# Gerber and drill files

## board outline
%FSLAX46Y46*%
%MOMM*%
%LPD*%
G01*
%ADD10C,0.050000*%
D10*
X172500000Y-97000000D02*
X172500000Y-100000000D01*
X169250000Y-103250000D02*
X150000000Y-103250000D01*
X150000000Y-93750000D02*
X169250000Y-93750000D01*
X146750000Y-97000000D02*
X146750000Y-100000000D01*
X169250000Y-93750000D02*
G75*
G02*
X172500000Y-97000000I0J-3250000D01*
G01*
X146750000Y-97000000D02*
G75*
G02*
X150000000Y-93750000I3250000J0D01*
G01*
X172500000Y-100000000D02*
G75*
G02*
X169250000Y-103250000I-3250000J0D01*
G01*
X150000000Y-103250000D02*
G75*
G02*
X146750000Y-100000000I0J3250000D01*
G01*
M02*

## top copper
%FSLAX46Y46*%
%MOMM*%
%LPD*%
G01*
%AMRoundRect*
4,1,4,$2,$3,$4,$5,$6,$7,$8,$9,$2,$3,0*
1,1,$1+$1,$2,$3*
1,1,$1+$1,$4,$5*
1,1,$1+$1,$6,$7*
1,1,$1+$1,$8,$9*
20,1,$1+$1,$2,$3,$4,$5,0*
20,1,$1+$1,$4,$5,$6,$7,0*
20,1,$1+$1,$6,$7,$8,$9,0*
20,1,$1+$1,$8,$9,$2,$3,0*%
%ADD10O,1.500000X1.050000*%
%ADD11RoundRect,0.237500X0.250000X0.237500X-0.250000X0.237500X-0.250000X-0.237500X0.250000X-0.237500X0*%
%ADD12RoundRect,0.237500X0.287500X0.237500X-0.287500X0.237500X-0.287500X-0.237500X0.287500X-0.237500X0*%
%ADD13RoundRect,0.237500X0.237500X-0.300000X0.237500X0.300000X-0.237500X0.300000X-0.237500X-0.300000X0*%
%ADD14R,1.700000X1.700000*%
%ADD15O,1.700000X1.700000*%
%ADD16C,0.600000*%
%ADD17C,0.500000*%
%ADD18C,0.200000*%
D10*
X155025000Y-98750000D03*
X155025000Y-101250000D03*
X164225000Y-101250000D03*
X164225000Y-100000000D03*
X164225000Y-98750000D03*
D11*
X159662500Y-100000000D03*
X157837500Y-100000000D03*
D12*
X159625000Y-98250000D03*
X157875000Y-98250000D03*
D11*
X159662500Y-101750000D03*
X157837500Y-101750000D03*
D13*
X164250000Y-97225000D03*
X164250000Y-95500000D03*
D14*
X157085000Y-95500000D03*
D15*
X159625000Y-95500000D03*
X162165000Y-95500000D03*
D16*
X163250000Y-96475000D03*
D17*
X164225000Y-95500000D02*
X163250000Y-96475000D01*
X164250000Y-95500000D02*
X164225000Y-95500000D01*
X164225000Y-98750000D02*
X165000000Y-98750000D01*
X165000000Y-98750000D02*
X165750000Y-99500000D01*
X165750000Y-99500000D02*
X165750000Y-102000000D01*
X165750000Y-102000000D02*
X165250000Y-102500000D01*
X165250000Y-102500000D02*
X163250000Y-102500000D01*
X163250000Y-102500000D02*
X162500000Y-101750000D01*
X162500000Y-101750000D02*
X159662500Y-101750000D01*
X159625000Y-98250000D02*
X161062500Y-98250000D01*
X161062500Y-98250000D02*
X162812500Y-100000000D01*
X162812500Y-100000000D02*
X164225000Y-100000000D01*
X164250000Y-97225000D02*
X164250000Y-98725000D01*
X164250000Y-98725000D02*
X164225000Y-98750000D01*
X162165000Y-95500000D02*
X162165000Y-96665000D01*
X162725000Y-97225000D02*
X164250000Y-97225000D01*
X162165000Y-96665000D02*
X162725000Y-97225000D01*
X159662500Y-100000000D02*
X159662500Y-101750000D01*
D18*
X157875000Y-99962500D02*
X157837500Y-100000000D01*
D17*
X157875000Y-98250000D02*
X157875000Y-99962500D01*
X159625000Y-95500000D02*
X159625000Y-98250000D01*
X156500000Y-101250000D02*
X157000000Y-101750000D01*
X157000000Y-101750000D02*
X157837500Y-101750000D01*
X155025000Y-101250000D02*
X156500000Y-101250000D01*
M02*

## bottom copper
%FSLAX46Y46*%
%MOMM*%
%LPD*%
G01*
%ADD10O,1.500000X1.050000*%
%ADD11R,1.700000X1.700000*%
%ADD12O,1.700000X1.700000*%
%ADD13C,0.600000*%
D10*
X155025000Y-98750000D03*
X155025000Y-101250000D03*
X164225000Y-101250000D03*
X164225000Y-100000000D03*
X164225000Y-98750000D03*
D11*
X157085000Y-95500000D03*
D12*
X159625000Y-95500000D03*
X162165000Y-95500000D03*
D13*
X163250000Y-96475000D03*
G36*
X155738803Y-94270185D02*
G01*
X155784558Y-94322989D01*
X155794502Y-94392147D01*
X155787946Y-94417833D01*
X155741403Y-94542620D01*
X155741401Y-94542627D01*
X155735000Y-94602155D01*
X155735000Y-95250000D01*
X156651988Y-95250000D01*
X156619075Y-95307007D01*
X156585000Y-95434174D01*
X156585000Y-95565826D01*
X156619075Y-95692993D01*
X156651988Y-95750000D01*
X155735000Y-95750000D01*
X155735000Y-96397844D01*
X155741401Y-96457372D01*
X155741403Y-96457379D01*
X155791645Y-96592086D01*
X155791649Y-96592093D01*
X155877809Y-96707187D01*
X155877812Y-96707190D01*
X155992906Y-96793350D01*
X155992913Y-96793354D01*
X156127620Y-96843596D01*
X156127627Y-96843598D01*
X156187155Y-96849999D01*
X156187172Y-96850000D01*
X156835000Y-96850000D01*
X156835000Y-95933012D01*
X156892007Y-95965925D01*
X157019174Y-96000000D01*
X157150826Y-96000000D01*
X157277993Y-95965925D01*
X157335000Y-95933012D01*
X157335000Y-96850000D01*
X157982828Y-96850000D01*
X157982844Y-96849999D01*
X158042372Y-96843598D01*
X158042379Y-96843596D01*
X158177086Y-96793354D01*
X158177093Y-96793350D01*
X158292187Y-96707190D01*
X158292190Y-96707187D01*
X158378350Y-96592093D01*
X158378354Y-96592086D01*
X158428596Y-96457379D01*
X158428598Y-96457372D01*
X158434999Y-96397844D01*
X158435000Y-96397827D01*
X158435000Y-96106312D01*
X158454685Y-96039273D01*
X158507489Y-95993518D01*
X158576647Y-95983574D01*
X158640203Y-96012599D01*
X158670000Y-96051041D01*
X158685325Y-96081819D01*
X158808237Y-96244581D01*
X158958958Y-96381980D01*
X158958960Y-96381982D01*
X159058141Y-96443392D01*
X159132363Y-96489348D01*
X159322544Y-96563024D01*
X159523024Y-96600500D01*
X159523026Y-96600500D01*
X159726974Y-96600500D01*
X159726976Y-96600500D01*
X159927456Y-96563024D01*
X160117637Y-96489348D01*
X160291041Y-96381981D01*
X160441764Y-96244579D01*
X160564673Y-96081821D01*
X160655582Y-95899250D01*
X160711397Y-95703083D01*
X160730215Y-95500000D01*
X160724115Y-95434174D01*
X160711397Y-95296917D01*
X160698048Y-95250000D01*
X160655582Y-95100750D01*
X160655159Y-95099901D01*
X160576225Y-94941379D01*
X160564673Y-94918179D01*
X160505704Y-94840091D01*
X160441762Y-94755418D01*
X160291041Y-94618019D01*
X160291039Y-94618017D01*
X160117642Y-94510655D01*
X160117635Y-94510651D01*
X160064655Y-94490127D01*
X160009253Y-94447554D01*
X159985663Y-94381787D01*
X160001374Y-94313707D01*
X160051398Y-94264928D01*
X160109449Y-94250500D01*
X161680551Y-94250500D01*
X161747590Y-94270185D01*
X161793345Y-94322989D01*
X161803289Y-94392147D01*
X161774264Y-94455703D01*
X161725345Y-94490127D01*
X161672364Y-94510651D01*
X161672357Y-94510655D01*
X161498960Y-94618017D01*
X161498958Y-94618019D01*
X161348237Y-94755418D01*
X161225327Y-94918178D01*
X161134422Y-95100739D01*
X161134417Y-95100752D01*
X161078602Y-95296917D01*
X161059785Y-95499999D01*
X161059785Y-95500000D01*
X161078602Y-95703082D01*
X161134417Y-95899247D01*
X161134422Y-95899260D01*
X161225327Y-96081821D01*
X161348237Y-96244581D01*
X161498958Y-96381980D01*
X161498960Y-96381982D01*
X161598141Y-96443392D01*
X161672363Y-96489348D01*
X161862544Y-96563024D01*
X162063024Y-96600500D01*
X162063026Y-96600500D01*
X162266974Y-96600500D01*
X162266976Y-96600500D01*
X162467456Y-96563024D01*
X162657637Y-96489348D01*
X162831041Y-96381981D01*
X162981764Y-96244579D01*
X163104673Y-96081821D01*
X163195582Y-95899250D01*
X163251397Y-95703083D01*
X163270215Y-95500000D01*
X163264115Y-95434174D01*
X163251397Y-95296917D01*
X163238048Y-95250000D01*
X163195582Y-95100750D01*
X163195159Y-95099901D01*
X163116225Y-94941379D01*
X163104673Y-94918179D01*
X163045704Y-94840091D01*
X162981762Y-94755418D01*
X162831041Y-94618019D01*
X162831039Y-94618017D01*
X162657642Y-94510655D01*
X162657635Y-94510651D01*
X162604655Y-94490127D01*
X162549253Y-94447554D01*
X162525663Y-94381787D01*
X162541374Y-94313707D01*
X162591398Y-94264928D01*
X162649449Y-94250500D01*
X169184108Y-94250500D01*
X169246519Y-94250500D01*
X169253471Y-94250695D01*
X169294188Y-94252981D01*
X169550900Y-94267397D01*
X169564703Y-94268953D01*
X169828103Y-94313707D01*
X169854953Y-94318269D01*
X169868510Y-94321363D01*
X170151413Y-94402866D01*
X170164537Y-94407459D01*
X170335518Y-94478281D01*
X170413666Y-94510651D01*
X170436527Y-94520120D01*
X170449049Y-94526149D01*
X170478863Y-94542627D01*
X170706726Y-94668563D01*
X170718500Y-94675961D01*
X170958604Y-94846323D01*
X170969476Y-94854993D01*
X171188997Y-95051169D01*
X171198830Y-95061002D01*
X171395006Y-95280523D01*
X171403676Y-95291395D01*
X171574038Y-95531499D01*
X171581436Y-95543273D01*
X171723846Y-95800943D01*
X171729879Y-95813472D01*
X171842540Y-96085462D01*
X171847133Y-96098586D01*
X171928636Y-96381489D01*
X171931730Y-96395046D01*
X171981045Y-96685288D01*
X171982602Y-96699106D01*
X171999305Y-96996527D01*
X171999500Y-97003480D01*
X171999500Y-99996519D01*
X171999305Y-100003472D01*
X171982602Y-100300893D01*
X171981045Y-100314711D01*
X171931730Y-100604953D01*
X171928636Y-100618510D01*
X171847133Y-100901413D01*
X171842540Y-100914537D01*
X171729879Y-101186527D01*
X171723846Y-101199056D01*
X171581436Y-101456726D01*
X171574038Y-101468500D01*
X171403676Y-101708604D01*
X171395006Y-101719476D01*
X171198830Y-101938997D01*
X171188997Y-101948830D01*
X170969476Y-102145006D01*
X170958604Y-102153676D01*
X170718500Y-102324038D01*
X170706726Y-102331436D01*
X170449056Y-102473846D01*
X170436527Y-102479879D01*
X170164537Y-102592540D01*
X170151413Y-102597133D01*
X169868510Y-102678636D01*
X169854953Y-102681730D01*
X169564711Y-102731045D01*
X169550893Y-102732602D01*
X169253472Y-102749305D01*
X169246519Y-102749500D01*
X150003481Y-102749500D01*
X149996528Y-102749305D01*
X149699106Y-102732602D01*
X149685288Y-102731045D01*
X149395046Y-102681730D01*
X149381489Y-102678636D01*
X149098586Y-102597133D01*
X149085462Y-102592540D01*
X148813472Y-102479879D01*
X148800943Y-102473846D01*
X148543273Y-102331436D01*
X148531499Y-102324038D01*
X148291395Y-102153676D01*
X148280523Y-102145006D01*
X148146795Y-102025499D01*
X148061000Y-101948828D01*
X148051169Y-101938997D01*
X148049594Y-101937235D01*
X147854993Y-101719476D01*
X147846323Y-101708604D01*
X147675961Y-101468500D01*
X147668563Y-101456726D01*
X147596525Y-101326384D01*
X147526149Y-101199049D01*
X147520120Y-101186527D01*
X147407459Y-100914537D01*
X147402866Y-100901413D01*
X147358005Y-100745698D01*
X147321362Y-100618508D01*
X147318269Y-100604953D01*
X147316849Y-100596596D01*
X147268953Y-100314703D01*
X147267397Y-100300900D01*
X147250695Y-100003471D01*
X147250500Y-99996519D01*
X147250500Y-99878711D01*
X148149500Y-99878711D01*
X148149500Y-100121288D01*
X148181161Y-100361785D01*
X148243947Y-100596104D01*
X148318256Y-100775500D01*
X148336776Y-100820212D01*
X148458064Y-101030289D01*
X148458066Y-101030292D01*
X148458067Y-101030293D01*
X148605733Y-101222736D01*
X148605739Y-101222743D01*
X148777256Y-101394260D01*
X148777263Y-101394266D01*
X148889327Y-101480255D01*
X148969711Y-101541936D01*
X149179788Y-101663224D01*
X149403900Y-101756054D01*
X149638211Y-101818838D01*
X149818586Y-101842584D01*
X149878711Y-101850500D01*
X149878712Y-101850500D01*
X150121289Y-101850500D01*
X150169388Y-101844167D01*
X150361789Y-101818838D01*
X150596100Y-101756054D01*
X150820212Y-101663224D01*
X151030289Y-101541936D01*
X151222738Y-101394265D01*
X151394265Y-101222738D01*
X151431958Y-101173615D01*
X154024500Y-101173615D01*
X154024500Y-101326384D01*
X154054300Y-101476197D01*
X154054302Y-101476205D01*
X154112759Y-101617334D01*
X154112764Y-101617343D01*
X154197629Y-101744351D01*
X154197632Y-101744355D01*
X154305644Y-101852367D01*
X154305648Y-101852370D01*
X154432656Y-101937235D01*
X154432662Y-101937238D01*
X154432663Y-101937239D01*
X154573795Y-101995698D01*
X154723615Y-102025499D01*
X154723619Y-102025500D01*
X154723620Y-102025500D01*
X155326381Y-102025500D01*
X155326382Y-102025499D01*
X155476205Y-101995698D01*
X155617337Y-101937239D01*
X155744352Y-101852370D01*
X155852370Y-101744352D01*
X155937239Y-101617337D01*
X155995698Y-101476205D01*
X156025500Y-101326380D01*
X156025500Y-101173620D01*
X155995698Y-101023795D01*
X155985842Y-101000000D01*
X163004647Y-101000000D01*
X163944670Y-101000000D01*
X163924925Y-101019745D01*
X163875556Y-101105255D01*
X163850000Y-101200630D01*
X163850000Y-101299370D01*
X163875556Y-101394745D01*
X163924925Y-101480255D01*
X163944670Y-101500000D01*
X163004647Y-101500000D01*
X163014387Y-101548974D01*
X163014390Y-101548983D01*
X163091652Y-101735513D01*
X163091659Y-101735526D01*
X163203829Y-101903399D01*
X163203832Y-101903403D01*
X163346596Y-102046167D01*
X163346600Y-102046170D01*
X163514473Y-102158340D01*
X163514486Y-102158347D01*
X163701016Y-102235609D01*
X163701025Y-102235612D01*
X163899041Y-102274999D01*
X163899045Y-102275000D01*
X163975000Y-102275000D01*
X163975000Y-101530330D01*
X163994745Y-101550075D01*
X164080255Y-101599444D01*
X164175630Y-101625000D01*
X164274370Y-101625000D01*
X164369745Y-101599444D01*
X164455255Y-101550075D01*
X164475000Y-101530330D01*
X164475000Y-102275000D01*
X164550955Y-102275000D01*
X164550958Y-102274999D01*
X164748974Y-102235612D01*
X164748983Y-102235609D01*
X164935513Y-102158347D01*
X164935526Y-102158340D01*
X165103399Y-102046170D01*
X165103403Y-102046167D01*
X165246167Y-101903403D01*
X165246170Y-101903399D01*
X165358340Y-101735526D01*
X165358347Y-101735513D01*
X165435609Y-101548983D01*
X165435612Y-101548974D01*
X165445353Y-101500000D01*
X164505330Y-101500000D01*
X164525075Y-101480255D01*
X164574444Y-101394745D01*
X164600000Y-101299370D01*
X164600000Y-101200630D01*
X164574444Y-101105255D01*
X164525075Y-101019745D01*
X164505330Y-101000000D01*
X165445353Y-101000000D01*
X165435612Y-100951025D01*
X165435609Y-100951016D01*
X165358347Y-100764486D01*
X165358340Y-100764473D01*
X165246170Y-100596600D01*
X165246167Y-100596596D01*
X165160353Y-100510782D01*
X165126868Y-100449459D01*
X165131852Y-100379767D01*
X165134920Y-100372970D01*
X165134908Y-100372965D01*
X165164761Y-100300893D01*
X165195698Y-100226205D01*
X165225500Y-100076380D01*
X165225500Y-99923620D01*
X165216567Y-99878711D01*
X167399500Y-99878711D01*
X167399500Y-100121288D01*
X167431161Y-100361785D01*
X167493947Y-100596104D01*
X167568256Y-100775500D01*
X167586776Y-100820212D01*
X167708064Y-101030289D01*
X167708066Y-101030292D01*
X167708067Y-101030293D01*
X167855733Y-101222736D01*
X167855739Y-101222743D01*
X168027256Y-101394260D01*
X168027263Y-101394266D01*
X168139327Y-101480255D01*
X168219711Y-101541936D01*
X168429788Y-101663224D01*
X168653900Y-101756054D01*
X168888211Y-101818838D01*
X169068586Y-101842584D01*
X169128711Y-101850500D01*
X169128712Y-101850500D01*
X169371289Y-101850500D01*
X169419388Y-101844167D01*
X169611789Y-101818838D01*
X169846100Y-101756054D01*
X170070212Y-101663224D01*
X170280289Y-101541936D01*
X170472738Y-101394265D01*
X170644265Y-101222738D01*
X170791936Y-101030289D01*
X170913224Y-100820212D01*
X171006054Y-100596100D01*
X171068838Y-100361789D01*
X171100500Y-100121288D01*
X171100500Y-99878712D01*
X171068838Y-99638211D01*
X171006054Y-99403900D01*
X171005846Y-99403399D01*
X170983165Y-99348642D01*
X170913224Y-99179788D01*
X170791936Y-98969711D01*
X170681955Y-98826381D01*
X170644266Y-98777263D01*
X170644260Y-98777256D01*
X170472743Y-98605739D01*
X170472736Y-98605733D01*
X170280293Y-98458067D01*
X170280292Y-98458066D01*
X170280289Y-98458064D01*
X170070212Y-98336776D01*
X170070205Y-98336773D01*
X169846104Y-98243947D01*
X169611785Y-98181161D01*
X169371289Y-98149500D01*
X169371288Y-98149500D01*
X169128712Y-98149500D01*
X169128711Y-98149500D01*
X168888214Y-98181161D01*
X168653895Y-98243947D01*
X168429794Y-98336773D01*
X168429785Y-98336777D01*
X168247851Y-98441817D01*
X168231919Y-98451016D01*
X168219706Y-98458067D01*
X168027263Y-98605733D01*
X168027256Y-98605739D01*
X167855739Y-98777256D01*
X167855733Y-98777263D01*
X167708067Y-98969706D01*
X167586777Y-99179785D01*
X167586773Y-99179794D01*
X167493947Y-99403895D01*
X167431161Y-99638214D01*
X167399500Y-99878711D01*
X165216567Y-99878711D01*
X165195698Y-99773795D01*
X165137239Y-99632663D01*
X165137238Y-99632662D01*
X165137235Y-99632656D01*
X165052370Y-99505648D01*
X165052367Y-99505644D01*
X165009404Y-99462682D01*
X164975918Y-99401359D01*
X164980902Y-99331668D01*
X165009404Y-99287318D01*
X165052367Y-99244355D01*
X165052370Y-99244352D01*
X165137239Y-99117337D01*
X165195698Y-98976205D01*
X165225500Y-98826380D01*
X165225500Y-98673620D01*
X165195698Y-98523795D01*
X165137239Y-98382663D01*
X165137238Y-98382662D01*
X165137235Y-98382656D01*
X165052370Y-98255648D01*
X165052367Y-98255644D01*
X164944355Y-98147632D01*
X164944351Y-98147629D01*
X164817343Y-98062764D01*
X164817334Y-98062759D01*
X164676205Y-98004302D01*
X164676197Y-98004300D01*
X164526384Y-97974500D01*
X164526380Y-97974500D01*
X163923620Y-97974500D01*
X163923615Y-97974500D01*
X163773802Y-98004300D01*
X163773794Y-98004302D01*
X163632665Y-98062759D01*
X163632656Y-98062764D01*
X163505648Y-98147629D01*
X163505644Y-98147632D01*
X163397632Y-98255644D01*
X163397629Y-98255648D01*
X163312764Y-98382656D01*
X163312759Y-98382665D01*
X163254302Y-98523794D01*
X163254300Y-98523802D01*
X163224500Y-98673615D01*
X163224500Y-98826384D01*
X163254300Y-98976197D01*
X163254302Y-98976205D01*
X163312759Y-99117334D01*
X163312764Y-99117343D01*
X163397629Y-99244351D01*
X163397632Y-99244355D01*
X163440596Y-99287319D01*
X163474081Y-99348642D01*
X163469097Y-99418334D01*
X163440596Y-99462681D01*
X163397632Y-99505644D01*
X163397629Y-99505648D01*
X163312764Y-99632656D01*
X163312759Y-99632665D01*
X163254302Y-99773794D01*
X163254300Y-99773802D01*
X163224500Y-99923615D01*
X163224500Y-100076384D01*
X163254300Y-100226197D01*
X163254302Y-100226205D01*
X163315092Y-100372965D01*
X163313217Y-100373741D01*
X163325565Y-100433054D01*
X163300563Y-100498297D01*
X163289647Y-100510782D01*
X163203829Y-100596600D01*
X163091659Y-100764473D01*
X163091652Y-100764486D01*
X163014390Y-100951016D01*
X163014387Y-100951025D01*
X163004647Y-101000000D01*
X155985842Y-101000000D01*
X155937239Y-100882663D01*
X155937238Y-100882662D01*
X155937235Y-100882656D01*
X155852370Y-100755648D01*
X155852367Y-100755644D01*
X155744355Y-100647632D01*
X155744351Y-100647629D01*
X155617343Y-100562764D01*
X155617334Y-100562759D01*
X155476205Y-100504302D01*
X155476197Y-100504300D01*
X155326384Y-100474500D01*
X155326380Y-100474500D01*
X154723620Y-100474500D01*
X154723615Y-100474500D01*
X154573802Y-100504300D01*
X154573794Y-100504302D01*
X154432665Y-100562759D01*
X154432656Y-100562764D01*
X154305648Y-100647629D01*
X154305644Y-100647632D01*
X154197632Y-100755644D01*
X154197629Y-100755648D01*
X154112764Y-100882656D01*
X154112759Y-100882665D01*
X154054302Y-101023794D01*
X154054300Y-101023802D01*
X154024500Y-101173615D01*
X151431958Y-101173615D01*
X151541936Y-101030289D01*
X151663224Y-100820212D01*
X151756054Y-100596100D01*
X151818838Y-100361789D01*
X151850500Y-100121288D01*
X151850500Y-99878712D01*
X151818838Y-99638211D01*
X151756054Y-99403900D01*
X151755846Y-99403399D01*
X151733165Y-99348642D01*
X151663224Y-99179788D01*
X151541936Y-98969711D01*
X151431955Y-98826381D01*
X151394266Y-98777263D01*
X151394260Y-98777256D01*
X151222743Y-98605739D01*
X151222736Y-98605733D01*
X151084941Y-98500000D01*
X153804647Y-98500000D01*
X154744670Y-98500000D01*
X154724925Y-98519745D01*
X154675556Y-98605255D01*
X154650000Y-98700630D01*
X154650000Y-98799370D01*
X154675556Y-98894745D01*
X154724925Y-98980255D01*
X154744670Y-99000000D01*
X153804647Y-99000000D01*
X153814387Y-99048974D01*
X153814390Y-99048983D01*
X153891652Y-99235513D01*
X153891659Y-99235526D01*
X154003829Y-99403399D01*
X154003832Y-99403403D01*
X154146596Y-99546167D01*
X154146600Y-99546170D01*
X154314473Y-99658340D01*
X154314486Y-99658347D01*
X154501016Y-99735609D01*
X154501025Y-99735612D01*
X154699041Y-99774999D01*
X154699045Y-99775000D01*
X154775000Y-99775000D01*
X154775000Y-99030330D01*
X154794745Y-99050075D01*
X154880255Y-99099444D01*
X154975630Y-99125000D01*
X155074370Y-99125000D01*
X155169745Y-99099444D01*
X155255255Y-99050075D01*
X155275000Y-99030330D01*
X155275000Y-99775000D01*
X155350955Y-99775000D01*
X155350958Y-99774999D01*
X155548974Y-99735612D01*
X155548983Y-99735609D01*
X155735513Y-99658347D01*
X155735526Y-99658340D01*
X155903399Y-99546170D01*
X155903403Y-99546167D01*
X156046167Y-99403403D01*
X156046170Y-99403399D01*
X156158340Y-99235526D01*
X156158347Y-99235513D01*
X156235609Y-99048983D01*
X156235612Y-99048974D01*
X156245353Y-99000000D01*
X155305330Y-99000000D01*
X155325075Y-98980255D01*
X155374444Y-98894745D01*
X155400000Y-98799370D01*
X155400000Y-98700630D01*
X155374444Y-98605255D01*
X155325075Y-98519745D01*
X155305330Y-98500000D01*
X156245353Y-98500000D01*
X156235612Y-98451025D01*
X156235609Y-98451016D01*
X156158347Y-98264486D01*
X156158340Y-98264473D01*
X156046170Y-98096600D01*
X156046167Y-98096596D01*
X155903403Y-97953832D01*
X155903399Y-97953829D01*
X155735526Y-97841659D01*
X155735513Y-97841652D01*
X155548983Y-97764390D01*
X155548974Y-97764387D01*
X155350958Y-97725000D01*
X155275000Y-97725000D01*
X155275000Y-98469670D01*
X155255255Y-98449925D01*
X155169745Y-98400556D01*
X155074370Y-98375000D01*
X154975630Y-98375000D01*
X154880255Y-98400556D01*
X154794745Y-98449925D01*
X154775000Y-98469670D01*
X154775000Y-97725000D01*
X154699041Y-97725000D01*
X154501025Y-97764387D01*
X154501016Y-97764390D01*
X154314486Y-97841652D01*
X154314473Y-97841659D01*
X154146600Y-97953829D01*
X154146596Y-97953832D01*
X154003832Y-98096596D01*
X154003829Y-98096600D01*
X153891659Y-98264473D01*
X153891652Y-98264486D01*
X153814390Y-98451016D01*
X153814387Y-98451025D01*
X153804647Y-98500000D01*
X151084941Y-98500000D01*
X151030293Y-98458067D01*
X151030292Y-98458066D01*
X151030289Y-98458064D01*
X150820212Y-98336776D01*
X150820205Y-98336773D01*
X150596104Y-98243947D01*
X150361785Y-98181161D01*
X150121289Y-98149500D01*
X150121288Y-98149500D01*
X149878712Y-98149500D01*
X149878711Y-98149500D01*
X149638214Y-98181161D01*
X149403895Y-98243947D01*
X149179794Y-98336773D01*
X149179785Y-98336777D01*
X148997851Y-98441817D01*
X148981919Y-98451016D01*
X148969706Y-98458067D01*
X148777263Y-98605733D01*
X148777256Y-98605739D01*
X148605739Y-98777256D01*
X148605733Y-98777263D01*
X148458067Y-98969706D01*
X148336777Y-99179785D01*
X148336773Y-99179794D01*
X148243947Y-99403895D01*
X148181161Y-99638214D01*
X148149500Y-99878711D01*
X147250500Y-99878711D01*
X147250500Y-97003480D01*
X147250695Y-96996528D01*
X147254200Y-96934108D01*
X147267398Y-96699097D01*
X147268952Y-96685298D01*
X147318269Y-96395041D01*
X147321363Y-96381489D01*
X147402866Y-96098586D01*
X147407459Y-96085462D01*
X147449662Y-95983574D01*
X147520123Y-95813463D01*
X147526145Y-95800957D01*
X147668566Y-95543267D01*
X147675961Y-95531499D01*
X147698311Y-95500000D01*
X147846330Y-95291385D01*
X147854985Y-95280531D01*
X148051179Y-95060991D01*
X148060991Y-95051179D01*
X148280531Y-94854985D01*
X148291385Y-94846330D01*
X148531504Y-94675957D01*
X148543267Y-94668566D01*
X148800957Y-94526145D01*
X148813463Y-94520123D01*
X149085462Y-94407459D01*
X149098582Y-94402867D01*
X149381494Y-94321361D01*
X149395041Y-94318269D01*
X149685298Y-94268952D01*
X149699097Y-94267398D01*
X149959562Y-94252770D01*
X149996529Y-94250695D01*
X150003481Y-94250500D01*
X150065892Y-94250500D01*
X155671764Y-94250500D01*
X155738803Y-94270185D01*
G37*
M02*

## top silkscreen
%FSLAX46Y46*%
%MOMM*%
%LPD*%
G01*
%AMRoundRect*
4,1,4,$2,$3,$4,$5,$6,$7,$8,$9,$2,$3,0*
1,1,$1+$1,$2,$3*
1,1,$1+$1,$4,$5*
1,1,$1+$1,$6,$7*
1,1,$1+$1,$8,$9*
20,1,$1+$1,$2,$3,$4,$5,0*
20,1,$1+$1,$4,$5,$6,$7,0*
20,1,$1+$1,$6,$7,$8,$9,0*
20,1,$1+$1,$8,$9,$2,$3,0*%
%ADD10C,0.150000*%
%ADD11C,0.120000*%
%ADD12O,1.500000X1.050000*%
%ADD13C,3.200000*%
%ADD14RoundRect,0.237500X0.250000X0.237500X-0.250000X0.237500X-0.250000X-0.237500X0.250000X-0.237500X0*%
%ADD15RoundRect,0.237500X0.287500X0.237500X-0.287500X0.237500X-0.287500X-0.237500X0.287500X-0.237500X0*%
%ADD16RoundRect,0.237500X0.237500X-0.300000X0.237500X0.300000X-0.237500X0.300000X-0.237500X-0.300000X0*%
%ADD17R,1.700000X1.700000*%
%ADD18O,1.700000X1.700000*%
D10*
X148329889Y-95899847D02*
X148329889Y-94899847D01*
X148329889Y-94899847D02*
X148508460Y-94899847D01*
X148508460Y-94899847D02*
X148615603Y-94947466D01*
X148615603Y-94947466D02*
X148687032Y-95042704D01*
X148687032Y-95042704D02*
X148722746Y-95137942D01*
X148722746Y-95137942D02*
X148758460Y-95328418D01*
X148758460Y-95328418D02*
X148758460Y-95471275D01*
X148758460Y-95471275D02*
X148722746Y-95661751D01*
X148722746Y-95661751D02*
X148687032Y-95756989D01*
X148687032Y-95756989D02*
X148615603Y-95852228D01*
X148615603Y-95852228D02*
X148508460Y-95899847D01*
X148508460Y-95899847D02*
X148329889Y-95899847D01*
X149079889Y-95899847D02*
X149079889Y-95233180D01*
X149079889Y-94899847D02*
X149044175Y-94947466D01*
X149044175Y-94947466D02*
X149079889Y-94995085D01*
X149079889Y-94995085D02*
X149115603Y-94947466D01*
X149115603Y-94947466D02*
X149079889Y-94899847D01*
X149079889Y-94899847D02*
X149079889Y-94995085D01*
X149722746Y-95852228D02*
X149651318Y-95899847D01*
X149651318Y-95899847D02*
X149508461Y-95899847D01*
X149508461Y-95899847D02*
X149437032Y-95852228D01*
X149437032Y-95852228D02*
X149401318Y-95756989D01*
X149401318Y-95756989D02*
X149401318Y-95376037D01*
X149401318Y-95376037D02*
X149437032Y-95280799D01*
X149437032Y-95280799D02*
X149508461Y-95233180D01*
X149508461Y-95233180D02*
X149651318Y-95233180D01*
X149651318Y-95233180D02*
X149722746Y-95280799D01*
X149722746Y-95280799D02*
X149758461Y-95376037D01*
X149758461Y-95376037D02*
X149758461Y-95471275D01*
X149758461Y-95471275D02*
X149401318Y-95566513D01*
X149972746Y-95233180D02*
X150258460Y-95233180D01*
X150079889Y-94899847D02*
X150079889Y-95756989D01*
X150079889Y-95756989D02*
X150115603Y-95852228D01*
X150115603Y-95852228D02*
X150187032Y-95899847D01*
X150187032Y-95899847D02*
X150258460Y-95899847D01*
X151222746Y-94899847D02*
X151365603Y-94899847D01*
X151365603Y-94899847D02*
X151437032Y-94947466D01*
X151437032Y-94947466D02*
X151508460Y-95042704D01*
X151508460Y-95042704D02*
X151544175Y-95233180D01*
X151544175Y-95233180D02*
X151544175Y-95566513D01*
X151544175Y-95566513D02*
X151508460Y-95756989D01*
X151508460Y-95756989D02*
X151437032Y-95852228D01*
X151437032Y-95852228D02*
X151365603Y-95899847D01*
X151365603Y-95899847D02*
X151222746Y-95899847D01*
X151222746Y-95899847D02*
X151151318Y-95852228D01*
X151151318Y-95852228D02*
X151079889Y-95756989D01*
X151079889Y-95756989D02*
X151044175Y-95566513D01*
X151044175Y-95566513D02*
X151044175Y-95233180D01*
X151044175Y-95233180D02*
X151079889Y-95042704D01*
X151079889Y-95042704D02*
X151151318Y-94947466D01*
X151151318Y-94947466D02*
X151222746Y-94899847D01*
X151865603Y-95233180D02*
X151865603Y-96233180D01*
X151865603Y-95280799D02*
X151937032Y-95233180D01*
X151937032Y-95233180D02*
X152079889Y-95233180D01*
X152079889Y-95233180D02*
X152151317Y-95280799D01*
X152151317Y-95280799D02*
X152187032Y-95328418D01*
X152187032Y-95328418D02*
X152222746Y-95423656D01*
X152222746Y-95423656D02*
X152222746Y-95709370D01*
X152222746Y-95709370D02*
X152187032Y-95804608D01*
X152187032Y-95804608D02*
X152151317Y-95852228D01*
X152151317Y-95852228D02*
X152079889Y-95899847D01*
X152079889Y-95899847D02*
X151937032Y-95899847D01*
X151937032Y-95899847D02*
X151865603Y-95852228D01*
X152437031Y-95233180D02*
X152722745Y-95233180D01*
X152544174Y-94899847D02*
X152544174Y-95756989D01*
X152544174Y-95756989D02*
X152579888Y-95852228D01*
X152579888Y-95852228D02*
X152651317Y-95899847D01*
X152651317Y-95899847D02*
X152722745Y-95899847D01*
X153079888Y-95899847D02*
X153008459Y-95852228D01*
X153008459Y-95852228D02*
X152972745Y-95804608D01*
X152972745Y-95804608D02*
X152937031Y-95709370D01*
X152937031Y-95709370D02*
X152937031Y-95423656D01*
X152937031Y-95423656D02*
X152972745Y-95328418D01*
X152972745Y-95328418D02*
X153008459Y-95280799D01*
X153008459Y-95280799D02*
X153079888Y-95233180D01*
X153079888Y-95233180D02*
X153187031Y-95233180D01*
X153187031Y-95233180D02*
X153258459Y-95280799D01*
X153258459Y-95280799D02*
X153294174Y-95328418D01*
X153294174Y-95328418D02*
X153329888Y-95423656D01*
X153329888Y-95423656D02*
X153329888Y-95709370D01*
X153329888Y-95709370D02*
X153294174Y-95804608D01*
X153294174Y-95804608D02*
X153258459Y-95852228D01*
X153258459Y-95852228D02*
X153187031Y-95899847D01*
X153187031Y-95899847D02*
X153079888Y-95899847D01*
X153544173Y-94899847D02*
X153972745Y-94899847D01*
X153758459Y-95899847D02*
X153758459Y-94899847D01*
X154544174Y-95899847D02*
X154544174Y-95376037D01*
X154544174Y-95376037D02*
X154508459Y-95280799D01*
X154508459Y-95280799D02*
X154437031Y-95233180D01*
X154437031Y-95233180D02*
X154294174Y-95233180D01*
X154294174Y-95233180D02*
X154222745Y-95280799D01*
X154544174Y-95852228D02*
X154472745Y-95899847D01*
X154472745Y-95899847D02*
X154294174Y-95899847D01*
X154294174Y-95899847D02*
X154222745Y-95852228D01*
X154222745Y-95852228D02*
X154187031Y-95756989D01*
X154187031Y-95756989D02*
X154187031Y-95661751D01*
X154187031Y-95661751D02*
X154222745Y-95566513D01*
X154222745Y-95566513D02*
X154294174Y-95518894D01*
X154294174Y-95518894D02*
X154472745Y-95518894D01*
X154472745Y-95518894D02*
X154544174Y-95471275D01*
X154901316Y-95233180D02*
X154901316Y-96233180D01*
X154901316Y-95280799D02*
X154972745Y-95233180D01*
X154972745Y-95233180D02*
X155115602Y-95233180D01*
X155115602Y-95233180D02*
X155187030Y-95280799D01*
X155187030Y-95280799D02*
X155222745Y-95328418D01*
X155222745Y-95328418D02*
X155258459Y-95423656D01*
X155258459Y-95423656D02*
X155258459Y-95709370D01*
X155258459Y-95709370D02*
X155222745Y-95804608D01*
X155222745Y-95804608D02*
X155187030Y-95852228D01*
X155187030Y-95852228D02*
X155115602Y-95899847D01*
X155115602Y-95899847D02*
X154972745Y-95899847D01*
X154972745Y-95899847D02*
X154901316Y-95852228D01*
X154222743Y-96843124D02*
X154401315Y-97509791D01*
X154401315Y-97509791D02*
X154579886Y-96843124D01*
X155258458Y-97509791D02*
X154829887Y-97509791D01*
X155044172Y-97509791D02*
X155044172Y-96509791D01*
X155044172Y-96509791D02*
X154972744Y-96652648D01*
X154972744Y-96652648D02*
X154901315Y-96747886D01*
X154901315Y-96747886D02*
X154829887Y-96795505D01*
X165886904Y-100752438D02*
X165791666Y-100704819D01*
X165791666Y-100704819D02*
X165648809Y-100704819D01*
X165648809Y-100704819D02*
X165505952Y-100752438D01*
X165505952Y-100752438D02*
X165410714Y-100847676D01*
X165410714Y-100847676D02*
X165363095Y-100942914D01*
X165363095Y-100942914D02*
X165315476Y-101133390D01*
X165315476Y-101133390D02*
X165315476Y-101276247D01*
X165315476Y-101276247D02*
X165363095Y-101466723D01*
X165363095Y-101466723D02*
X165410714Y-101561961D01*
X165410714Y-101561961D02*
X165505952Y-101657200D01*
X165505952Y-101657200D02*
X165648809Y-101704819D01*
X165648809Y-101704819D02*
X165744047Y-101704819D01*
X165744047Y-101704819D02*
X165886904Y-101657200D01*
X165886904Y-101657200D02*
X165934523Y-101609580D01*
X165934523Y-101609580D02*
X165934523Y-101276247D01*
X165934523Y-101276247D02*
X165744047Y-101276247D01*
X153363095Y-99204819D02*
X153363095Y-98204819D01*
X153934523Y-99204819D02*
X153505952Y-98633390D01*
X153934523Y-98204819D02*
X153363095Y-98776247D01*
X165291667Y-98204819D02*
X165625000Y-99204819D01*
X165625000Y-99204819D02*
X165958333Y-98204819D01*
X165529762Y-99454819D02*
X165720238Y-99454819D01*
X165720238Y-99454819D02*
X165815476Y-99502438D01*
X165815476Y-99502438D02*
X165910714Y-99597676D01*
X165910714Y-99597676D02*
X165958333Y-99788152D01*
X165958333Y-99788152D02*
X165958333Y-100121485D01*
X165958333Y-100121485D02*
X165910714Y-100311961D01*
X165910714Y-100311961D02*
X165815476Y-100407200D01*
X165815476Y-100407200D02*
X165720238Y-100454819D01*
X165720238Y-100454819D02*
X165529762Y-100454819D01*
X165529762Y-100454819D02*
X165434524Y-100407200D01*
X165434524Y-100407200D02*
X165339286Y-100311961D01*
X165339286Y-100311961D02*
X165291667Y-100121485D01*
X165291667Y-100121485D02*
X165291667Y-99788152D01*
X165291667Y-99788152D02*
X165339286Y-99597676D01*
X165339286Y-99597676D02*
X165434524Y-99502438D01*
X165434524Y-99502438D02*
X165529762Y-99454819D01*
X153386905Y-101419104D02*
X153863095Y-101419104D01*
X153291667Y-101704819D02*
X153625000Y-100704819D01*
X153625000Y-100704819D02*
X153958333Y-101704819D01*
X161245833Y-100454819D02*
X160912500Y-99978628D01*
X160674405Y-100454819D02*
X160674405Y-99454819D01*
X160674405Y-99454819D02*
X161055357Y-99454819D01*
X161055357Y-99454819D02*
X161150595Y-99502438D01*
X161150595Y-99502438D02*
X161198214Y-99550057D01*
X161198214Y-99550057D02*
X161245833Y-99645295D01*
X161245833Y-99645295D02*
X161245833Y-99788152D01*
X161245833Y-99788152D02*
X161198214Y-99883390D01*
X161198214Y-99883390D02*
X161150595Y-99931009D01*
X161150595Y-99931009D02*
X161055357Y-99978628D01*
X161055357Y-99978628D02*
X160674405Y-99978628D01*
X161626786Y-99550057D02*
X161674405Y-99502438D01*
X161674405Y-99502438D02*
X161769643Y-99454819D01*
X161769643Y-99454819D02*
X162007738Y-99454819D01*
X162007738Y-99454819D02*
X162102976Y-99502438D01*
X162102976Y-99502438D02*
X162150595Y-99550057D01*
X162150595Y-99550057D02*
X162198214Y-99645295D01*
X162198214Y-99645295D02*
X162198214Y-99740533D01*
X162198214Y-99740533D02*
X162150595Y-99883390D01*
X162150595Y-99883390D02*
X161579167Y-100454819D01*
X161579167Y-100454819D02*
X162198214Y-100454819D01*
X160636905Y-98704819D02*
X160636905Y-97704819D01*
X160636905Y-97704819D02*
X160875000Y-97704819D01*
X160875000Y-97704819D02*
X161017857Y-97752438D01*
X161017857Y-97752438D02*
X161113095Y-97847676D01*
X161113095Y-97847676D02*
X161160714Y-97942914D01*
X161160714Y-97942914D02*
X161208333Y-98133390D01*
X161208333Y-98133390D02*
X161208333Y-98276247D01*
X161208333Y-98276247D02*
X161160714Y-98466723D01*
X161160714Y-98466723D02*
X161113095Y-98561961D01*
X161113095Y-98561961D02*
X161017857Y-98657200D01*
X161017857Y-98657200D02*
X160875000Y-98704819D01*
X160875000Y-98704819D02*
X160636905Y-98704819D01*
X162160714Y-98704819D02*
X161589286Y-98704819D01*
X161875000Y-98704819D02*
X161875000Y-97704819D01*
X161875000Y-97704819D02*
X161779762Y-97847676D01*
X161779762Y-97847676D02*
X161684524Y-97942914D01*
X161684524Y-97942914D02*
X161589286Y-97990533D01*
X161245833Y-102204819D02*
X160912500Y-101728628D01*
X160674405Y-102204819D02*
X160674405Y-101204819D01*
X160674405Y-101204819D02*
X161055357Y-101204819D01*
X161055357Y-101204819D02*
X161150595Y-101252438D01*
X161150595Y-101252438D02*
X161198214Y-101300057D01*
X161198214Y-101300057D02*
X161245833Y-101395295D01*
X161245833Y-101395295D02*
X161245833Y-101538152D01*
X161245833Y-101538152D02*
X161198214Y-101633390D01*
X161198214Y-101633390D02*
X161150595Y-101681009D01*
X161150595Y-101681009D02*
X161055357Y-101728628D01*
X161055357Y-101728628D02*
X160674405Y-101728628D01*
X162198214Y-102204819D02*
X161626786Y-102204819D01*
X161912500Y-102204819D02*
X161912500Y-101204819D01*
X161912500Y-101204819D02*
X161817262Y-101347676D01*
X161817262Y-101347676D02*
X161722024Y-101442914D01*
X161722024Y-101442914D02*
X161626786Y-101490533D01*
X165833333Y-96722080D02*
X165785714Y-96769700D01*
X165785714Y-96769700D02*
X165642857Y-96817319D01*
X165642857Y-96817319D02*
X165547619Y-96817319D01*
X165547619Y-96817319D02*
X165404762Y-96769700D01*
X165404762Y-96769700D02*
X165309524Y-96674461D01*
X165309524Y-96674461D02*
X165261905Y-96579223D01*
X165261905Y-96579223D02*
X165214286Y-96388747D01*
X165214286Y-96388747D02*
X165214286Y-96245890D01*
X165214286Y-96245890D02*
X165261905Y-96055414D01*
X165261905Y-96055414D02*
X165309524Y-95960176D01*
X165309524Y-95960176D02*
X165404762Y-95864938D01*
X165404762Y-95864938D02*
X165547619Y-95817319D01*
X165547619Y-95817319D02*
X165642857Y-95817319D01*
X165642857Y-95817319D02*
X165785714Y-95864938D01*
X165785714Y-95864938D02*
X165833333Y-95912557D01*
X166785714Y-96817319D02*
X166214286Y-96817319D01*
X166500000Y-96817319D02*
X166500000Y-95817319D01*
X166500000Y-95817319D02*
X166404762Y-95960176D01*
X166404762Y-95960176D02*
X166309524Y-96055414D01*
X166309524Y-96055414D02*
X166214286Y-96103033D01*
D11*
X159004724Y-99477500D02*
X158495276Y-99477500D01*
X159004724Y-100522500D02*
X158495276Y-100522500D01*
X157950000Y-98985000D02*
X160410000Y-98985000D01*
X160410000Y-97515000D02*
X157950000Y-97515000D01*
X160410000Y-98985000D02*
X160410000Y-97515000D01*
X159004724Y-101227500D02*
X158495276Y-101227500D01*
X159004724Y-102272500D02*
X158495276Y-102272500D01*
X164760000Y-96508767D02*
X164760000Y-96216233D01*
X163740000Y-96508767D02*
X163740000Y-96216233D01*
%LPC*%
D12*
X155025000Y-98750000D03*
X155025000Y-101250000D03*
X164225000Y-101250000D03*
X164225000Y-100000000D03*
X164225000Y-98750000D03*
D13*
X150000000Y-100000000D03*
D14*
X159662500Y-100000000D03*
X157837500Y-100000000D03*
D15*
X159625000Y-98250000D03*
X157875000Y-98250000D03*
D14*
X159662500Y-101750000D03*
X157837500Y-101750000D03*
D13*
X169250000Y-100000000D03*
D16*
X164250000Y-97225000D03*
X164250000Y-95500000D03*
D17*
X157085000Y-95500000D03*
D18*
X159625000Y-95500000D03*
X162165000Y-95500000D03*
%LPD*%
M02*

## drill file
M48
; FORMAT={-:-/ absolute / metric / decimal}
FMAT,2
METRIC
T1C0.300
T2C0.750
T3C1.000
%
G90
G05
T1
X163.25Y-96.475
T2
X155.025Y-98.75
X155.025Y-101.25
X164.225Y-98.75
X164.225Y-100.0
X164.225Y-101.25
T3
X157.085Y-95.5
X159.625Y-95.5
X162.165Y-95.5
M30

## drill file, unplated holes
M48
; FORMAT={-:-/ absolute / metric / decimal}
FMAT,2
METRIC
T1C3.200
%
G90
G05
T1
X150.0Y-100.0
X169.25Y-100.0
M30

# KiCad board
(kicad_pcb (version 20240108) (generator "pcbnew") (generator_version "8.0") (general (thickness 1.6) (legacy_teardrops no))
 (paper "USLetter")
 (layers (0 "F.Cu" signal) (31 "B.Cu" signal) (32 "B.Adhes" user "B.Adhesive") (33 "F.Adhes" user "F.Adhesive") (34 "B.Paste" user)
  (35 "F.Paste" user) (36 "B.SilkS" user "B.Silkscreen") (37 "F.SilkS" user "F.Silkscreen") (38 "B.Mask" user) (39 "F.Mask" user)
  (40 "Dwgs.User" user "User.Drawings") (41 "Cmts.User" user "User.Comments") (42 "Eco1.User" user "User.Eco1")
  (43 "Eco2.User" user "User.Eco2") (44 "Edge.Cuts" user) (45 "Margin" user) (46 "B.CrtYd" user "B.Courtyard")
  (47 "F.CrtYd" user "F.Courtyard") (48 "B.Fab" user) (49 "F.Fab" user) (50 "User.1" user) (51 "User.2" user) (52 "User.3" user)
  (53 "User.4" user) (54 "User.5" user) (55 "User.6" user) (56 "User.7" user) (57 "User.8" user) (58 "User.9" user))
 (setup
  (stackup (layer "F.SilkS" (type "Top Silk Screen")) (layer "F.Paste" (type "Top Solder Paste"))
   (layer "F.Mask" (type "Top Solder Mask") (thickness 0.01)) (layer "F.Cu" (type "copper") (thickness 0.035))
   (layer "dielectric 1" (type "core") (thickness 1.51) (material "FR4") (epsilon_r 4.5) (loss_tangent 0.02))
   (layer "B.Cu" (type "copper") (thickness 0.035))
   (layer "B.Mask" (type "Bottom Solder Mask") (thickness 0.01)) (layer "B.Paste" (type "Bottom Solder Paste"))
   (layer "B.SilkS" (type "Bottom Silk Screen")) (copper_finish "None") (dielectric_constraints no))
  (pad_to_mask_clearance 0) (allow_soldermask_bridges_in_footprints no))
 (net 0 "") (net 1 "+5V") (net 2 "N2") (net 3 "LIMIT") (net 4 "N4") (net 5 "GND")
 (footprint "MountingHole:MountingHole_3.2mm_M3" (layer "F.Cu") (at 150 100)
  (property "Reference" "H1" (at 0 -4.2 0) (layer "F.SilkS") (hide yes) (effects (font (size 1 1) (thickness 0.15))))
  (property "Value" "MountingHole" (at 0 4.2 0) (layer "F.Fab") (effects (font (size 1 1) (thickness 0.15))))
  (pad "" np_thru_hole circle (at 0 0) (size 3.2 3.2) (drill 3.2) (layers "F&B.Cu" "*.Mask")))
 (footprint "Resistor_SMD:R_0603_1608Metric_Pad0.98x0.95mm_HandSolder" (layer "F.Cu") (at 158.75 100 180)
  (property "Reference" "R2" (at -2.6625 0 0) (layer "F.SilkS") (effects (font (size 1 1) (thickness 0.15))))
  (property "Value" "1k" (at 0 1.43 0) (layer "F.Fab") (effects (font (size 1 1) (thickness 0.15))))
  (fp_line (start -0.254724 0.5225) (end 0.254724 0.5225) (stroke (width 0.12) (type solid)) (layer "F.SilkS"))
  (fp_line (start -0.254724 -0.5225) (end 0.254724 -0.5225) (stroke (width 0.12) (type solid)) (layer "F.SilkS"))
  (pad "1" smd roundrect (at -0.9125 0 180) (size 0.975 0.95) (layers "F.Cu" "F.Paste" "F.Mask") (roundrect_rratio 0.25) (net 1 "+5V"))
  (pad "2" smd roundrect (at 0.9125 0 180) (size 0.975 0.95) (layers "F.Cu" "F.Paste" "F.Mask") (roundrect_rratio 0.25) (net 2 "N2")))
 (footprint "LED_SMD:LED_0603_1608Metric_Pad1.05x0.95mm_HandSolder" (layer "F.Cu") (at 158.75 98.25 180)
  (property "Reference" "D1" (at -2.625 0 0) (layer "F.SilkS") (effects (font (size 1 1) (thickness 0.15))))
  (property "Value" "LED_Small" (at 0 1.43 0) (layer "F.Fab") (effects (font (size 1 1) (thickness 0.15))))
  (fp_line (start 0.8 -0.735) (end -1.66 -0.735) (stroke (width 0.12) (type solid)) (layer "F.SilkS"))
  (fp_line (start -1.66 0.735) (end 0.8 0.735) (stroke (width 0.12) (type solid)) (layer "F.SilkS"))
  (fp_line (start -1.66 -0.735) (end -1.66 0.735) (stroke (width 0.12) (type solid)) (layer "F.SilkS"))
  (pad "1" smd roundrect (at -0.875 0 180) (size 1.05 0.95) (layers "F.Cu" "F.Paste" "F.Mask") (roundrect_rratio 0.25) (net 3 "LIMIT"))
  (pad "2" smd roundrect (at 0.875 0 180) (size 1.05 0.95) (layers "F.Cu" "F.Paste" "F.Mask") (roundrect_rratio 0.25) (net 2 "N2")))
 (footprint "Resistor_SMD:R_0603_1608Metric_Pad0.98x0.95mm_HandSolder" (layer "F.Cu") (at 158.75 101.75 180)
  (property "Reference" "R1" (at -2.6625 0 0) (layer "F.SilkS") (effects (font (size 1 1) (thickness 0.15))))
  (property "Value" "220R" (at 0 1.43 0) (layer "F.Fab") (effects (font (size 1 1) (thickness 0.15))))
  (fp_line (start -0.254724 0.5225) (end 0.254724 0.5225) (stroke (width 0.12) (type solid)) (layer "F.SilkS"))
  (fp_line (start -0.254724 -0.5225) (end 0.254724 -0.5225) (stroke (width 0.12) (type solid)) (layer "F.SilkS"))
  (pad "1" smd roundrect (at -0.9125 0 180) (size 0.975 0.95) (layers "F.Cu" "F.Paste" "F.Mask") (roundrect_rratio 0.25) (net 1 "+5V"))
  (pad "2" smd roundrect (at 0.9125 0 180) (size 0.975 0.95) (layers "F.Cu" "F.Paste" "F.Mask") (roundrect_rratio 0.25) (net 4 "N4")))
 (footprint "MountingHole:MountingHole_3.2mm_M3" (layer "F.Cu") (at 169.25 100)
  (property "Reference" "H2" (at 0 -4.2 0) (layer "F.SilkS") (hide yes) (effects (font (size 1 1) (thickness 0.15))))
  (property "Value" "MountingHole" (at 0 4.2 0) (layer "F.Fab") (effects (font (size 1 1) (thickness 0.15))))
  (pad "" np_thru_hole circle (at 0 0) (size 3.2 3.2) (drill 3.2) (layers "F&B.Cu" "*.Mask")))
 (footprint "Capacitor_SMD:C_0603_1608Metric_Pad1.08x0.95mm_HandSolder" (layer "F.Cu") (at 164.25 96.3625 90)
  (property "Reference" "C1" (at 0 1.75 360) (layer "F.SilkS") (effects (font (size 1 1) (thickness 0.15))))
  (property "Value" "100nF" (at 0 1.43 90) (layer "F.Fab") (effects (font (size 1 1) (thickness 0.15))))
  (fp_line (start -0.146267 -0.51) (end 0.146267 -0.51) (stroke (width 0.12) (type solid)) (layer "F.SilkS"))
  (fp_line (start -0.146267 0.51) (end 0.146267 0.51) (stroke (width 0.12) (type solid)) (layer "F.SilkS"))
  (pad "1" smd roundrect (at -0.8625 0 90) (size 1.075 0.95) (layers "F.Cu" "F.Paste" "F.Mask") (roundrect_rratio 0.25) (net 1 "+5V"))
  (pad "2" smd roundrect (at 0.8625 0 90) (size 1.075 0.95) (layers "F.Cu" "F.Paste" "F.Mask") (roundrect_rratio 0.25) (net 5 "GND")))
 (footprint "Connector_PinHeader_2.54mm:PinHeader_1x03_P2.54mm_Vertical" (layer "B.Cu") (at 157.085 95.5 -90)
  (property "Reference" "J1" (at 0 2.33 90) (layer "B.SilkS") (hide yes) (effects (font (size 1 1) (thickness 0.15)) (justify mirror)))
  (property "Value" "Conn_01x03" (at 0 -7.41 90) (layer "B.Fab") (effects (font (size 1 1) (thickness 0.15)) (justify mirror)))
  (pad "1" thru_hole rect (at 0 0 270) (size 1.7 1.7) (drill 1) (layers "*.Cu" "*.Mask") (remove_unused_layers no) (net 5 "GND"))
  (pad "2" thru_hole oval (at 0 -2.54 270) (size 1.7 1.7) (drill 1) (layers "*.Cu" "*.Mask") (remove_unused_layers no) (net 3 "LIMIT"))
  (pad "3" thru_hole oval (at 0 -5.08 270) (size 1.7 1.7) (drill 1) (layers "*.Cu" "*.Mask") (remove_unused_layers no) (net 1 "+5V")))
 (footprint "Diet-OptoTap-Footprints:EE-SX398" (layer "B.Cu") (at 159.625 100 180)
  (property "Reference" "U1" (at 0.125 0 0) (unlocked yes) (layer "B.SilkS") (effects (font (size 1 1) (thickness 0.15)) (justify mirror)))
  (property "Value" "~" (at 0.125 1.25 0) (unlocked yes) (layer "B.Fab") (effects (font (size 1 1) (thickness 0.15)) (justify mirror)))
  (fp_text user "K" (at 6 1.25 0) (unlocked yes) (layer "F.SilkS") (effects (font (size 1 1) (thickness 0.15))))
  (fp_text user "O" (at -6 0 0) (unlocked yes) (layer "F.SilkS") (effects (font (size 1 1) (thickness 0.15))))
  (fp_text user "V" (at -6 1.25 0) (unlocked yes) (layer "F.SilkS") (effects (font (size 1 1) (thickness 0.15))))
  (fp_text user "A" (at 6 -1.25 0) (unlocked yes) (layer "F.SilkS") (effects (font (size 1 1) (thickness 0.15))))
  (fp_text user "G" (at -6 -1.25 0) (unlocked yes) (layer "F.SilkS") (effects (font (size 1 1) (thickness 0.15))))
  (pad "1" thru_hole oval (at 4.6 1.25 180) (size 1.5 1.05) (drill 0.75) (layers "*.Cu" "*.Mask") (remove_unused_layers no) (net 5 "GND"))
  (pad "2" thru_hole oval (at 4.6 -1.25 180) (size 1.5 1.05) (drill 0.75) (layers "*.Cu" "*.Mask") (remove_unused_layers no) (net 4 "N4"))
  (pad "3" thru_hole oval (at -4.6 -1.25 180) (size 1.5 1.05) (drill 0.75) (layers "*.Cu" "*.Mask") (remove_unused_layers no) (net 5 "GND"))
  (pad "4" thru_hole oval (at -4.6 0 180) (size 1.5 1.05) (drill 0.75) (layers "*.Cu" "*.Mask") (remove_unused_layers no) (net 3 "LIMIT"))
  (pad "5" thru_hole oval (at -4.6 1.25 180) (size 1.5 1.05) (drill 0.75) (layers "*.Cu" "*.Mask") (remove_unused_layers no) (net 1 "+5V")))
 (gr_line (start 172.5 97) (end 172.5 100) (stroke (width 0.05) (type default)) (layer "Edge.Cuts"))
 (gr_line (start 169.25 103.25) (end 150 103.25) (stroke (width 0.05) (type default)) (layer "Edge.Cuts"))
 (gr_line (start 150 93.75) (end 169.25 93.75) (stroke (width 0.05) (type default)) (layer "Edge.Cuts"))
 (gr_line (start 146.75 97) (end 146.75 100) (stroke (width 0.05) (type default)) (layer "Edge.Cuts"))
 (gr_arc (start 169.25 93.75) (mid 171.548097 94.701903) (end 172.5 97) (stroke (width 0.05) (type default)) (layer "Edge.Cuts"))
 (gr_arc (start 146.75 97) (mid 147.701903 94.701903) (end 150 93.75) (stroke (width 0.05) (type default)) (layer "Edge.Cuts"))
 (gr_arc (start 172.5 100) (mid 171.548097 102.298097) (end 169.25 103.25) (stroke (width 0.05) (type default)) (layer "Edge.Cuts"))
 (gr_arc (start 150 103.25) (mid 147.701903 102.298097) (end 146.75 100) (stroke (width 0.05) (type default)) (layer "Edge.Cuts"))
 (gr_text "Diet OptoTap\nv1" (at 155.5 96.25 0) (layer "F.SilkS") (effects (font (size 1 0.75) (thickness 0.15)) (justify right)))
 (segment (start 164.225 95.5) (end 163.25 96.475) (width 0.5) (layer "F.Cu") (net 5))
 (segment (start 164.25 95.5) (end 164.225 95.5) (width 0.5) (layer "F.Cu") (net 5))
 (via (at 163.25 96.475) (size 0.6) (drill 0.3) (layers "F.Cu" "B.Cu") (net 5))
 (segment (start 163.25 102.5) (end 162.5 101.75) (width 0.5) (layer "F.Cu") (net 1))
 (segment (start 162.5 101.75) (end 159.6625 101.75) (width 0.5) (layer "F.Cu") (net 1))
 (segment (start 165.75 102) (end 165.25 102.5) (width 0.5) (layer "F.Cu") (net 1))
 (segment (start 165 98.75) (end 165.75 99.5) (width 0.5) (layer "F.Cu") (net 1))
 (segment (start 164.25 97.225) (end 164.25 98.725) (width 0.5) (layer "F.Cu") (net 1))
 (segment (start 164.225 98.75) (end 165 98.75) (width 0.5) (layer "F.Cu") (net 1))
 (segment (start 165.75 99.5) (end 165.75 102) (width 0.5) (layer "F.Cu") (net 1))
 (segment (start 165.25 102.5) (end 163.25 102.5) (width 0.5) (layer "F.Cu") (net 1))
 (segment (start 159.6625 100) (end 159.6625 101.75) (width 0.5) (layer "F.Cu") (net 1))
 (segment (start 162.165 96.665) (end 162.725 97.225) (width 0.5) (layer "F.Cu") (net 1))
 (segment (start 164.25 98.725) (end 164.225 98.75) (width 0.5) (layer "F.Cu") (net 1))
 (segment (start 162.165 95.5) (end 162.165 96.665) (width 0.5) (layer "F.Cu") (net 1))
 (segment (start 162.725 97.225) (end 164.25 97.225) (width 0.5) (layer "F.Cu") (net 1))
 (segment (start 157.875 99.9625) (end 157.8375 100) (width 0.2) (layer "F.Cu") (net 2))
 (segment (start 157.875 98.25) (end 157.875 99.9625) (width 0.5) (layer "F.Cu") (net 2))
 (segment (start 162.8125 100) (end 164.225 100) (width 0.5) (layer "F.Cu") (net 3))
 (segment (start 159.625 95.5) (end 159.625 98.25) (width 0.5) (layer "F.Cu") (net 3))
 (segment (start 161.0625 98.25) (end 162.8125 100) (width 0.5) (layer "F.Cu") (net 3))
 (segment (start 159.625 98.25) (end 161.0625 98.25) (width 0.5) (layer "F.Cu") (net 3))
 (segment (start 156.5 101.25) (end 157 101.75) (width 0.5) (layer "F.Cu") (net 4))
 (segment (start 157 101.75) (end 157.8375 101.75) (width 0.5) (layer "F.Cu") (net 4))
 (segment (start 155.025 101.25) (end 156.5 101.25) (width 0.5) (layer "F.Cu") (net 4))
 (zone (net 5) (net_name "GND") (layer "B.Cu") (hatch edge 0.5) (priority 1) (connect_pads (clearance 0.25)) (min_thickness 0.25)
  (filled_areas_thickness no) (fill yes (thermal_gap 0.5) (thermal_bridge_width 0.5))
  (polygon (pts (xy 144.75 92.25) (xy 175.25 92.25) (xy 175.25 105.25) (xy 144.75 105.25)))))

